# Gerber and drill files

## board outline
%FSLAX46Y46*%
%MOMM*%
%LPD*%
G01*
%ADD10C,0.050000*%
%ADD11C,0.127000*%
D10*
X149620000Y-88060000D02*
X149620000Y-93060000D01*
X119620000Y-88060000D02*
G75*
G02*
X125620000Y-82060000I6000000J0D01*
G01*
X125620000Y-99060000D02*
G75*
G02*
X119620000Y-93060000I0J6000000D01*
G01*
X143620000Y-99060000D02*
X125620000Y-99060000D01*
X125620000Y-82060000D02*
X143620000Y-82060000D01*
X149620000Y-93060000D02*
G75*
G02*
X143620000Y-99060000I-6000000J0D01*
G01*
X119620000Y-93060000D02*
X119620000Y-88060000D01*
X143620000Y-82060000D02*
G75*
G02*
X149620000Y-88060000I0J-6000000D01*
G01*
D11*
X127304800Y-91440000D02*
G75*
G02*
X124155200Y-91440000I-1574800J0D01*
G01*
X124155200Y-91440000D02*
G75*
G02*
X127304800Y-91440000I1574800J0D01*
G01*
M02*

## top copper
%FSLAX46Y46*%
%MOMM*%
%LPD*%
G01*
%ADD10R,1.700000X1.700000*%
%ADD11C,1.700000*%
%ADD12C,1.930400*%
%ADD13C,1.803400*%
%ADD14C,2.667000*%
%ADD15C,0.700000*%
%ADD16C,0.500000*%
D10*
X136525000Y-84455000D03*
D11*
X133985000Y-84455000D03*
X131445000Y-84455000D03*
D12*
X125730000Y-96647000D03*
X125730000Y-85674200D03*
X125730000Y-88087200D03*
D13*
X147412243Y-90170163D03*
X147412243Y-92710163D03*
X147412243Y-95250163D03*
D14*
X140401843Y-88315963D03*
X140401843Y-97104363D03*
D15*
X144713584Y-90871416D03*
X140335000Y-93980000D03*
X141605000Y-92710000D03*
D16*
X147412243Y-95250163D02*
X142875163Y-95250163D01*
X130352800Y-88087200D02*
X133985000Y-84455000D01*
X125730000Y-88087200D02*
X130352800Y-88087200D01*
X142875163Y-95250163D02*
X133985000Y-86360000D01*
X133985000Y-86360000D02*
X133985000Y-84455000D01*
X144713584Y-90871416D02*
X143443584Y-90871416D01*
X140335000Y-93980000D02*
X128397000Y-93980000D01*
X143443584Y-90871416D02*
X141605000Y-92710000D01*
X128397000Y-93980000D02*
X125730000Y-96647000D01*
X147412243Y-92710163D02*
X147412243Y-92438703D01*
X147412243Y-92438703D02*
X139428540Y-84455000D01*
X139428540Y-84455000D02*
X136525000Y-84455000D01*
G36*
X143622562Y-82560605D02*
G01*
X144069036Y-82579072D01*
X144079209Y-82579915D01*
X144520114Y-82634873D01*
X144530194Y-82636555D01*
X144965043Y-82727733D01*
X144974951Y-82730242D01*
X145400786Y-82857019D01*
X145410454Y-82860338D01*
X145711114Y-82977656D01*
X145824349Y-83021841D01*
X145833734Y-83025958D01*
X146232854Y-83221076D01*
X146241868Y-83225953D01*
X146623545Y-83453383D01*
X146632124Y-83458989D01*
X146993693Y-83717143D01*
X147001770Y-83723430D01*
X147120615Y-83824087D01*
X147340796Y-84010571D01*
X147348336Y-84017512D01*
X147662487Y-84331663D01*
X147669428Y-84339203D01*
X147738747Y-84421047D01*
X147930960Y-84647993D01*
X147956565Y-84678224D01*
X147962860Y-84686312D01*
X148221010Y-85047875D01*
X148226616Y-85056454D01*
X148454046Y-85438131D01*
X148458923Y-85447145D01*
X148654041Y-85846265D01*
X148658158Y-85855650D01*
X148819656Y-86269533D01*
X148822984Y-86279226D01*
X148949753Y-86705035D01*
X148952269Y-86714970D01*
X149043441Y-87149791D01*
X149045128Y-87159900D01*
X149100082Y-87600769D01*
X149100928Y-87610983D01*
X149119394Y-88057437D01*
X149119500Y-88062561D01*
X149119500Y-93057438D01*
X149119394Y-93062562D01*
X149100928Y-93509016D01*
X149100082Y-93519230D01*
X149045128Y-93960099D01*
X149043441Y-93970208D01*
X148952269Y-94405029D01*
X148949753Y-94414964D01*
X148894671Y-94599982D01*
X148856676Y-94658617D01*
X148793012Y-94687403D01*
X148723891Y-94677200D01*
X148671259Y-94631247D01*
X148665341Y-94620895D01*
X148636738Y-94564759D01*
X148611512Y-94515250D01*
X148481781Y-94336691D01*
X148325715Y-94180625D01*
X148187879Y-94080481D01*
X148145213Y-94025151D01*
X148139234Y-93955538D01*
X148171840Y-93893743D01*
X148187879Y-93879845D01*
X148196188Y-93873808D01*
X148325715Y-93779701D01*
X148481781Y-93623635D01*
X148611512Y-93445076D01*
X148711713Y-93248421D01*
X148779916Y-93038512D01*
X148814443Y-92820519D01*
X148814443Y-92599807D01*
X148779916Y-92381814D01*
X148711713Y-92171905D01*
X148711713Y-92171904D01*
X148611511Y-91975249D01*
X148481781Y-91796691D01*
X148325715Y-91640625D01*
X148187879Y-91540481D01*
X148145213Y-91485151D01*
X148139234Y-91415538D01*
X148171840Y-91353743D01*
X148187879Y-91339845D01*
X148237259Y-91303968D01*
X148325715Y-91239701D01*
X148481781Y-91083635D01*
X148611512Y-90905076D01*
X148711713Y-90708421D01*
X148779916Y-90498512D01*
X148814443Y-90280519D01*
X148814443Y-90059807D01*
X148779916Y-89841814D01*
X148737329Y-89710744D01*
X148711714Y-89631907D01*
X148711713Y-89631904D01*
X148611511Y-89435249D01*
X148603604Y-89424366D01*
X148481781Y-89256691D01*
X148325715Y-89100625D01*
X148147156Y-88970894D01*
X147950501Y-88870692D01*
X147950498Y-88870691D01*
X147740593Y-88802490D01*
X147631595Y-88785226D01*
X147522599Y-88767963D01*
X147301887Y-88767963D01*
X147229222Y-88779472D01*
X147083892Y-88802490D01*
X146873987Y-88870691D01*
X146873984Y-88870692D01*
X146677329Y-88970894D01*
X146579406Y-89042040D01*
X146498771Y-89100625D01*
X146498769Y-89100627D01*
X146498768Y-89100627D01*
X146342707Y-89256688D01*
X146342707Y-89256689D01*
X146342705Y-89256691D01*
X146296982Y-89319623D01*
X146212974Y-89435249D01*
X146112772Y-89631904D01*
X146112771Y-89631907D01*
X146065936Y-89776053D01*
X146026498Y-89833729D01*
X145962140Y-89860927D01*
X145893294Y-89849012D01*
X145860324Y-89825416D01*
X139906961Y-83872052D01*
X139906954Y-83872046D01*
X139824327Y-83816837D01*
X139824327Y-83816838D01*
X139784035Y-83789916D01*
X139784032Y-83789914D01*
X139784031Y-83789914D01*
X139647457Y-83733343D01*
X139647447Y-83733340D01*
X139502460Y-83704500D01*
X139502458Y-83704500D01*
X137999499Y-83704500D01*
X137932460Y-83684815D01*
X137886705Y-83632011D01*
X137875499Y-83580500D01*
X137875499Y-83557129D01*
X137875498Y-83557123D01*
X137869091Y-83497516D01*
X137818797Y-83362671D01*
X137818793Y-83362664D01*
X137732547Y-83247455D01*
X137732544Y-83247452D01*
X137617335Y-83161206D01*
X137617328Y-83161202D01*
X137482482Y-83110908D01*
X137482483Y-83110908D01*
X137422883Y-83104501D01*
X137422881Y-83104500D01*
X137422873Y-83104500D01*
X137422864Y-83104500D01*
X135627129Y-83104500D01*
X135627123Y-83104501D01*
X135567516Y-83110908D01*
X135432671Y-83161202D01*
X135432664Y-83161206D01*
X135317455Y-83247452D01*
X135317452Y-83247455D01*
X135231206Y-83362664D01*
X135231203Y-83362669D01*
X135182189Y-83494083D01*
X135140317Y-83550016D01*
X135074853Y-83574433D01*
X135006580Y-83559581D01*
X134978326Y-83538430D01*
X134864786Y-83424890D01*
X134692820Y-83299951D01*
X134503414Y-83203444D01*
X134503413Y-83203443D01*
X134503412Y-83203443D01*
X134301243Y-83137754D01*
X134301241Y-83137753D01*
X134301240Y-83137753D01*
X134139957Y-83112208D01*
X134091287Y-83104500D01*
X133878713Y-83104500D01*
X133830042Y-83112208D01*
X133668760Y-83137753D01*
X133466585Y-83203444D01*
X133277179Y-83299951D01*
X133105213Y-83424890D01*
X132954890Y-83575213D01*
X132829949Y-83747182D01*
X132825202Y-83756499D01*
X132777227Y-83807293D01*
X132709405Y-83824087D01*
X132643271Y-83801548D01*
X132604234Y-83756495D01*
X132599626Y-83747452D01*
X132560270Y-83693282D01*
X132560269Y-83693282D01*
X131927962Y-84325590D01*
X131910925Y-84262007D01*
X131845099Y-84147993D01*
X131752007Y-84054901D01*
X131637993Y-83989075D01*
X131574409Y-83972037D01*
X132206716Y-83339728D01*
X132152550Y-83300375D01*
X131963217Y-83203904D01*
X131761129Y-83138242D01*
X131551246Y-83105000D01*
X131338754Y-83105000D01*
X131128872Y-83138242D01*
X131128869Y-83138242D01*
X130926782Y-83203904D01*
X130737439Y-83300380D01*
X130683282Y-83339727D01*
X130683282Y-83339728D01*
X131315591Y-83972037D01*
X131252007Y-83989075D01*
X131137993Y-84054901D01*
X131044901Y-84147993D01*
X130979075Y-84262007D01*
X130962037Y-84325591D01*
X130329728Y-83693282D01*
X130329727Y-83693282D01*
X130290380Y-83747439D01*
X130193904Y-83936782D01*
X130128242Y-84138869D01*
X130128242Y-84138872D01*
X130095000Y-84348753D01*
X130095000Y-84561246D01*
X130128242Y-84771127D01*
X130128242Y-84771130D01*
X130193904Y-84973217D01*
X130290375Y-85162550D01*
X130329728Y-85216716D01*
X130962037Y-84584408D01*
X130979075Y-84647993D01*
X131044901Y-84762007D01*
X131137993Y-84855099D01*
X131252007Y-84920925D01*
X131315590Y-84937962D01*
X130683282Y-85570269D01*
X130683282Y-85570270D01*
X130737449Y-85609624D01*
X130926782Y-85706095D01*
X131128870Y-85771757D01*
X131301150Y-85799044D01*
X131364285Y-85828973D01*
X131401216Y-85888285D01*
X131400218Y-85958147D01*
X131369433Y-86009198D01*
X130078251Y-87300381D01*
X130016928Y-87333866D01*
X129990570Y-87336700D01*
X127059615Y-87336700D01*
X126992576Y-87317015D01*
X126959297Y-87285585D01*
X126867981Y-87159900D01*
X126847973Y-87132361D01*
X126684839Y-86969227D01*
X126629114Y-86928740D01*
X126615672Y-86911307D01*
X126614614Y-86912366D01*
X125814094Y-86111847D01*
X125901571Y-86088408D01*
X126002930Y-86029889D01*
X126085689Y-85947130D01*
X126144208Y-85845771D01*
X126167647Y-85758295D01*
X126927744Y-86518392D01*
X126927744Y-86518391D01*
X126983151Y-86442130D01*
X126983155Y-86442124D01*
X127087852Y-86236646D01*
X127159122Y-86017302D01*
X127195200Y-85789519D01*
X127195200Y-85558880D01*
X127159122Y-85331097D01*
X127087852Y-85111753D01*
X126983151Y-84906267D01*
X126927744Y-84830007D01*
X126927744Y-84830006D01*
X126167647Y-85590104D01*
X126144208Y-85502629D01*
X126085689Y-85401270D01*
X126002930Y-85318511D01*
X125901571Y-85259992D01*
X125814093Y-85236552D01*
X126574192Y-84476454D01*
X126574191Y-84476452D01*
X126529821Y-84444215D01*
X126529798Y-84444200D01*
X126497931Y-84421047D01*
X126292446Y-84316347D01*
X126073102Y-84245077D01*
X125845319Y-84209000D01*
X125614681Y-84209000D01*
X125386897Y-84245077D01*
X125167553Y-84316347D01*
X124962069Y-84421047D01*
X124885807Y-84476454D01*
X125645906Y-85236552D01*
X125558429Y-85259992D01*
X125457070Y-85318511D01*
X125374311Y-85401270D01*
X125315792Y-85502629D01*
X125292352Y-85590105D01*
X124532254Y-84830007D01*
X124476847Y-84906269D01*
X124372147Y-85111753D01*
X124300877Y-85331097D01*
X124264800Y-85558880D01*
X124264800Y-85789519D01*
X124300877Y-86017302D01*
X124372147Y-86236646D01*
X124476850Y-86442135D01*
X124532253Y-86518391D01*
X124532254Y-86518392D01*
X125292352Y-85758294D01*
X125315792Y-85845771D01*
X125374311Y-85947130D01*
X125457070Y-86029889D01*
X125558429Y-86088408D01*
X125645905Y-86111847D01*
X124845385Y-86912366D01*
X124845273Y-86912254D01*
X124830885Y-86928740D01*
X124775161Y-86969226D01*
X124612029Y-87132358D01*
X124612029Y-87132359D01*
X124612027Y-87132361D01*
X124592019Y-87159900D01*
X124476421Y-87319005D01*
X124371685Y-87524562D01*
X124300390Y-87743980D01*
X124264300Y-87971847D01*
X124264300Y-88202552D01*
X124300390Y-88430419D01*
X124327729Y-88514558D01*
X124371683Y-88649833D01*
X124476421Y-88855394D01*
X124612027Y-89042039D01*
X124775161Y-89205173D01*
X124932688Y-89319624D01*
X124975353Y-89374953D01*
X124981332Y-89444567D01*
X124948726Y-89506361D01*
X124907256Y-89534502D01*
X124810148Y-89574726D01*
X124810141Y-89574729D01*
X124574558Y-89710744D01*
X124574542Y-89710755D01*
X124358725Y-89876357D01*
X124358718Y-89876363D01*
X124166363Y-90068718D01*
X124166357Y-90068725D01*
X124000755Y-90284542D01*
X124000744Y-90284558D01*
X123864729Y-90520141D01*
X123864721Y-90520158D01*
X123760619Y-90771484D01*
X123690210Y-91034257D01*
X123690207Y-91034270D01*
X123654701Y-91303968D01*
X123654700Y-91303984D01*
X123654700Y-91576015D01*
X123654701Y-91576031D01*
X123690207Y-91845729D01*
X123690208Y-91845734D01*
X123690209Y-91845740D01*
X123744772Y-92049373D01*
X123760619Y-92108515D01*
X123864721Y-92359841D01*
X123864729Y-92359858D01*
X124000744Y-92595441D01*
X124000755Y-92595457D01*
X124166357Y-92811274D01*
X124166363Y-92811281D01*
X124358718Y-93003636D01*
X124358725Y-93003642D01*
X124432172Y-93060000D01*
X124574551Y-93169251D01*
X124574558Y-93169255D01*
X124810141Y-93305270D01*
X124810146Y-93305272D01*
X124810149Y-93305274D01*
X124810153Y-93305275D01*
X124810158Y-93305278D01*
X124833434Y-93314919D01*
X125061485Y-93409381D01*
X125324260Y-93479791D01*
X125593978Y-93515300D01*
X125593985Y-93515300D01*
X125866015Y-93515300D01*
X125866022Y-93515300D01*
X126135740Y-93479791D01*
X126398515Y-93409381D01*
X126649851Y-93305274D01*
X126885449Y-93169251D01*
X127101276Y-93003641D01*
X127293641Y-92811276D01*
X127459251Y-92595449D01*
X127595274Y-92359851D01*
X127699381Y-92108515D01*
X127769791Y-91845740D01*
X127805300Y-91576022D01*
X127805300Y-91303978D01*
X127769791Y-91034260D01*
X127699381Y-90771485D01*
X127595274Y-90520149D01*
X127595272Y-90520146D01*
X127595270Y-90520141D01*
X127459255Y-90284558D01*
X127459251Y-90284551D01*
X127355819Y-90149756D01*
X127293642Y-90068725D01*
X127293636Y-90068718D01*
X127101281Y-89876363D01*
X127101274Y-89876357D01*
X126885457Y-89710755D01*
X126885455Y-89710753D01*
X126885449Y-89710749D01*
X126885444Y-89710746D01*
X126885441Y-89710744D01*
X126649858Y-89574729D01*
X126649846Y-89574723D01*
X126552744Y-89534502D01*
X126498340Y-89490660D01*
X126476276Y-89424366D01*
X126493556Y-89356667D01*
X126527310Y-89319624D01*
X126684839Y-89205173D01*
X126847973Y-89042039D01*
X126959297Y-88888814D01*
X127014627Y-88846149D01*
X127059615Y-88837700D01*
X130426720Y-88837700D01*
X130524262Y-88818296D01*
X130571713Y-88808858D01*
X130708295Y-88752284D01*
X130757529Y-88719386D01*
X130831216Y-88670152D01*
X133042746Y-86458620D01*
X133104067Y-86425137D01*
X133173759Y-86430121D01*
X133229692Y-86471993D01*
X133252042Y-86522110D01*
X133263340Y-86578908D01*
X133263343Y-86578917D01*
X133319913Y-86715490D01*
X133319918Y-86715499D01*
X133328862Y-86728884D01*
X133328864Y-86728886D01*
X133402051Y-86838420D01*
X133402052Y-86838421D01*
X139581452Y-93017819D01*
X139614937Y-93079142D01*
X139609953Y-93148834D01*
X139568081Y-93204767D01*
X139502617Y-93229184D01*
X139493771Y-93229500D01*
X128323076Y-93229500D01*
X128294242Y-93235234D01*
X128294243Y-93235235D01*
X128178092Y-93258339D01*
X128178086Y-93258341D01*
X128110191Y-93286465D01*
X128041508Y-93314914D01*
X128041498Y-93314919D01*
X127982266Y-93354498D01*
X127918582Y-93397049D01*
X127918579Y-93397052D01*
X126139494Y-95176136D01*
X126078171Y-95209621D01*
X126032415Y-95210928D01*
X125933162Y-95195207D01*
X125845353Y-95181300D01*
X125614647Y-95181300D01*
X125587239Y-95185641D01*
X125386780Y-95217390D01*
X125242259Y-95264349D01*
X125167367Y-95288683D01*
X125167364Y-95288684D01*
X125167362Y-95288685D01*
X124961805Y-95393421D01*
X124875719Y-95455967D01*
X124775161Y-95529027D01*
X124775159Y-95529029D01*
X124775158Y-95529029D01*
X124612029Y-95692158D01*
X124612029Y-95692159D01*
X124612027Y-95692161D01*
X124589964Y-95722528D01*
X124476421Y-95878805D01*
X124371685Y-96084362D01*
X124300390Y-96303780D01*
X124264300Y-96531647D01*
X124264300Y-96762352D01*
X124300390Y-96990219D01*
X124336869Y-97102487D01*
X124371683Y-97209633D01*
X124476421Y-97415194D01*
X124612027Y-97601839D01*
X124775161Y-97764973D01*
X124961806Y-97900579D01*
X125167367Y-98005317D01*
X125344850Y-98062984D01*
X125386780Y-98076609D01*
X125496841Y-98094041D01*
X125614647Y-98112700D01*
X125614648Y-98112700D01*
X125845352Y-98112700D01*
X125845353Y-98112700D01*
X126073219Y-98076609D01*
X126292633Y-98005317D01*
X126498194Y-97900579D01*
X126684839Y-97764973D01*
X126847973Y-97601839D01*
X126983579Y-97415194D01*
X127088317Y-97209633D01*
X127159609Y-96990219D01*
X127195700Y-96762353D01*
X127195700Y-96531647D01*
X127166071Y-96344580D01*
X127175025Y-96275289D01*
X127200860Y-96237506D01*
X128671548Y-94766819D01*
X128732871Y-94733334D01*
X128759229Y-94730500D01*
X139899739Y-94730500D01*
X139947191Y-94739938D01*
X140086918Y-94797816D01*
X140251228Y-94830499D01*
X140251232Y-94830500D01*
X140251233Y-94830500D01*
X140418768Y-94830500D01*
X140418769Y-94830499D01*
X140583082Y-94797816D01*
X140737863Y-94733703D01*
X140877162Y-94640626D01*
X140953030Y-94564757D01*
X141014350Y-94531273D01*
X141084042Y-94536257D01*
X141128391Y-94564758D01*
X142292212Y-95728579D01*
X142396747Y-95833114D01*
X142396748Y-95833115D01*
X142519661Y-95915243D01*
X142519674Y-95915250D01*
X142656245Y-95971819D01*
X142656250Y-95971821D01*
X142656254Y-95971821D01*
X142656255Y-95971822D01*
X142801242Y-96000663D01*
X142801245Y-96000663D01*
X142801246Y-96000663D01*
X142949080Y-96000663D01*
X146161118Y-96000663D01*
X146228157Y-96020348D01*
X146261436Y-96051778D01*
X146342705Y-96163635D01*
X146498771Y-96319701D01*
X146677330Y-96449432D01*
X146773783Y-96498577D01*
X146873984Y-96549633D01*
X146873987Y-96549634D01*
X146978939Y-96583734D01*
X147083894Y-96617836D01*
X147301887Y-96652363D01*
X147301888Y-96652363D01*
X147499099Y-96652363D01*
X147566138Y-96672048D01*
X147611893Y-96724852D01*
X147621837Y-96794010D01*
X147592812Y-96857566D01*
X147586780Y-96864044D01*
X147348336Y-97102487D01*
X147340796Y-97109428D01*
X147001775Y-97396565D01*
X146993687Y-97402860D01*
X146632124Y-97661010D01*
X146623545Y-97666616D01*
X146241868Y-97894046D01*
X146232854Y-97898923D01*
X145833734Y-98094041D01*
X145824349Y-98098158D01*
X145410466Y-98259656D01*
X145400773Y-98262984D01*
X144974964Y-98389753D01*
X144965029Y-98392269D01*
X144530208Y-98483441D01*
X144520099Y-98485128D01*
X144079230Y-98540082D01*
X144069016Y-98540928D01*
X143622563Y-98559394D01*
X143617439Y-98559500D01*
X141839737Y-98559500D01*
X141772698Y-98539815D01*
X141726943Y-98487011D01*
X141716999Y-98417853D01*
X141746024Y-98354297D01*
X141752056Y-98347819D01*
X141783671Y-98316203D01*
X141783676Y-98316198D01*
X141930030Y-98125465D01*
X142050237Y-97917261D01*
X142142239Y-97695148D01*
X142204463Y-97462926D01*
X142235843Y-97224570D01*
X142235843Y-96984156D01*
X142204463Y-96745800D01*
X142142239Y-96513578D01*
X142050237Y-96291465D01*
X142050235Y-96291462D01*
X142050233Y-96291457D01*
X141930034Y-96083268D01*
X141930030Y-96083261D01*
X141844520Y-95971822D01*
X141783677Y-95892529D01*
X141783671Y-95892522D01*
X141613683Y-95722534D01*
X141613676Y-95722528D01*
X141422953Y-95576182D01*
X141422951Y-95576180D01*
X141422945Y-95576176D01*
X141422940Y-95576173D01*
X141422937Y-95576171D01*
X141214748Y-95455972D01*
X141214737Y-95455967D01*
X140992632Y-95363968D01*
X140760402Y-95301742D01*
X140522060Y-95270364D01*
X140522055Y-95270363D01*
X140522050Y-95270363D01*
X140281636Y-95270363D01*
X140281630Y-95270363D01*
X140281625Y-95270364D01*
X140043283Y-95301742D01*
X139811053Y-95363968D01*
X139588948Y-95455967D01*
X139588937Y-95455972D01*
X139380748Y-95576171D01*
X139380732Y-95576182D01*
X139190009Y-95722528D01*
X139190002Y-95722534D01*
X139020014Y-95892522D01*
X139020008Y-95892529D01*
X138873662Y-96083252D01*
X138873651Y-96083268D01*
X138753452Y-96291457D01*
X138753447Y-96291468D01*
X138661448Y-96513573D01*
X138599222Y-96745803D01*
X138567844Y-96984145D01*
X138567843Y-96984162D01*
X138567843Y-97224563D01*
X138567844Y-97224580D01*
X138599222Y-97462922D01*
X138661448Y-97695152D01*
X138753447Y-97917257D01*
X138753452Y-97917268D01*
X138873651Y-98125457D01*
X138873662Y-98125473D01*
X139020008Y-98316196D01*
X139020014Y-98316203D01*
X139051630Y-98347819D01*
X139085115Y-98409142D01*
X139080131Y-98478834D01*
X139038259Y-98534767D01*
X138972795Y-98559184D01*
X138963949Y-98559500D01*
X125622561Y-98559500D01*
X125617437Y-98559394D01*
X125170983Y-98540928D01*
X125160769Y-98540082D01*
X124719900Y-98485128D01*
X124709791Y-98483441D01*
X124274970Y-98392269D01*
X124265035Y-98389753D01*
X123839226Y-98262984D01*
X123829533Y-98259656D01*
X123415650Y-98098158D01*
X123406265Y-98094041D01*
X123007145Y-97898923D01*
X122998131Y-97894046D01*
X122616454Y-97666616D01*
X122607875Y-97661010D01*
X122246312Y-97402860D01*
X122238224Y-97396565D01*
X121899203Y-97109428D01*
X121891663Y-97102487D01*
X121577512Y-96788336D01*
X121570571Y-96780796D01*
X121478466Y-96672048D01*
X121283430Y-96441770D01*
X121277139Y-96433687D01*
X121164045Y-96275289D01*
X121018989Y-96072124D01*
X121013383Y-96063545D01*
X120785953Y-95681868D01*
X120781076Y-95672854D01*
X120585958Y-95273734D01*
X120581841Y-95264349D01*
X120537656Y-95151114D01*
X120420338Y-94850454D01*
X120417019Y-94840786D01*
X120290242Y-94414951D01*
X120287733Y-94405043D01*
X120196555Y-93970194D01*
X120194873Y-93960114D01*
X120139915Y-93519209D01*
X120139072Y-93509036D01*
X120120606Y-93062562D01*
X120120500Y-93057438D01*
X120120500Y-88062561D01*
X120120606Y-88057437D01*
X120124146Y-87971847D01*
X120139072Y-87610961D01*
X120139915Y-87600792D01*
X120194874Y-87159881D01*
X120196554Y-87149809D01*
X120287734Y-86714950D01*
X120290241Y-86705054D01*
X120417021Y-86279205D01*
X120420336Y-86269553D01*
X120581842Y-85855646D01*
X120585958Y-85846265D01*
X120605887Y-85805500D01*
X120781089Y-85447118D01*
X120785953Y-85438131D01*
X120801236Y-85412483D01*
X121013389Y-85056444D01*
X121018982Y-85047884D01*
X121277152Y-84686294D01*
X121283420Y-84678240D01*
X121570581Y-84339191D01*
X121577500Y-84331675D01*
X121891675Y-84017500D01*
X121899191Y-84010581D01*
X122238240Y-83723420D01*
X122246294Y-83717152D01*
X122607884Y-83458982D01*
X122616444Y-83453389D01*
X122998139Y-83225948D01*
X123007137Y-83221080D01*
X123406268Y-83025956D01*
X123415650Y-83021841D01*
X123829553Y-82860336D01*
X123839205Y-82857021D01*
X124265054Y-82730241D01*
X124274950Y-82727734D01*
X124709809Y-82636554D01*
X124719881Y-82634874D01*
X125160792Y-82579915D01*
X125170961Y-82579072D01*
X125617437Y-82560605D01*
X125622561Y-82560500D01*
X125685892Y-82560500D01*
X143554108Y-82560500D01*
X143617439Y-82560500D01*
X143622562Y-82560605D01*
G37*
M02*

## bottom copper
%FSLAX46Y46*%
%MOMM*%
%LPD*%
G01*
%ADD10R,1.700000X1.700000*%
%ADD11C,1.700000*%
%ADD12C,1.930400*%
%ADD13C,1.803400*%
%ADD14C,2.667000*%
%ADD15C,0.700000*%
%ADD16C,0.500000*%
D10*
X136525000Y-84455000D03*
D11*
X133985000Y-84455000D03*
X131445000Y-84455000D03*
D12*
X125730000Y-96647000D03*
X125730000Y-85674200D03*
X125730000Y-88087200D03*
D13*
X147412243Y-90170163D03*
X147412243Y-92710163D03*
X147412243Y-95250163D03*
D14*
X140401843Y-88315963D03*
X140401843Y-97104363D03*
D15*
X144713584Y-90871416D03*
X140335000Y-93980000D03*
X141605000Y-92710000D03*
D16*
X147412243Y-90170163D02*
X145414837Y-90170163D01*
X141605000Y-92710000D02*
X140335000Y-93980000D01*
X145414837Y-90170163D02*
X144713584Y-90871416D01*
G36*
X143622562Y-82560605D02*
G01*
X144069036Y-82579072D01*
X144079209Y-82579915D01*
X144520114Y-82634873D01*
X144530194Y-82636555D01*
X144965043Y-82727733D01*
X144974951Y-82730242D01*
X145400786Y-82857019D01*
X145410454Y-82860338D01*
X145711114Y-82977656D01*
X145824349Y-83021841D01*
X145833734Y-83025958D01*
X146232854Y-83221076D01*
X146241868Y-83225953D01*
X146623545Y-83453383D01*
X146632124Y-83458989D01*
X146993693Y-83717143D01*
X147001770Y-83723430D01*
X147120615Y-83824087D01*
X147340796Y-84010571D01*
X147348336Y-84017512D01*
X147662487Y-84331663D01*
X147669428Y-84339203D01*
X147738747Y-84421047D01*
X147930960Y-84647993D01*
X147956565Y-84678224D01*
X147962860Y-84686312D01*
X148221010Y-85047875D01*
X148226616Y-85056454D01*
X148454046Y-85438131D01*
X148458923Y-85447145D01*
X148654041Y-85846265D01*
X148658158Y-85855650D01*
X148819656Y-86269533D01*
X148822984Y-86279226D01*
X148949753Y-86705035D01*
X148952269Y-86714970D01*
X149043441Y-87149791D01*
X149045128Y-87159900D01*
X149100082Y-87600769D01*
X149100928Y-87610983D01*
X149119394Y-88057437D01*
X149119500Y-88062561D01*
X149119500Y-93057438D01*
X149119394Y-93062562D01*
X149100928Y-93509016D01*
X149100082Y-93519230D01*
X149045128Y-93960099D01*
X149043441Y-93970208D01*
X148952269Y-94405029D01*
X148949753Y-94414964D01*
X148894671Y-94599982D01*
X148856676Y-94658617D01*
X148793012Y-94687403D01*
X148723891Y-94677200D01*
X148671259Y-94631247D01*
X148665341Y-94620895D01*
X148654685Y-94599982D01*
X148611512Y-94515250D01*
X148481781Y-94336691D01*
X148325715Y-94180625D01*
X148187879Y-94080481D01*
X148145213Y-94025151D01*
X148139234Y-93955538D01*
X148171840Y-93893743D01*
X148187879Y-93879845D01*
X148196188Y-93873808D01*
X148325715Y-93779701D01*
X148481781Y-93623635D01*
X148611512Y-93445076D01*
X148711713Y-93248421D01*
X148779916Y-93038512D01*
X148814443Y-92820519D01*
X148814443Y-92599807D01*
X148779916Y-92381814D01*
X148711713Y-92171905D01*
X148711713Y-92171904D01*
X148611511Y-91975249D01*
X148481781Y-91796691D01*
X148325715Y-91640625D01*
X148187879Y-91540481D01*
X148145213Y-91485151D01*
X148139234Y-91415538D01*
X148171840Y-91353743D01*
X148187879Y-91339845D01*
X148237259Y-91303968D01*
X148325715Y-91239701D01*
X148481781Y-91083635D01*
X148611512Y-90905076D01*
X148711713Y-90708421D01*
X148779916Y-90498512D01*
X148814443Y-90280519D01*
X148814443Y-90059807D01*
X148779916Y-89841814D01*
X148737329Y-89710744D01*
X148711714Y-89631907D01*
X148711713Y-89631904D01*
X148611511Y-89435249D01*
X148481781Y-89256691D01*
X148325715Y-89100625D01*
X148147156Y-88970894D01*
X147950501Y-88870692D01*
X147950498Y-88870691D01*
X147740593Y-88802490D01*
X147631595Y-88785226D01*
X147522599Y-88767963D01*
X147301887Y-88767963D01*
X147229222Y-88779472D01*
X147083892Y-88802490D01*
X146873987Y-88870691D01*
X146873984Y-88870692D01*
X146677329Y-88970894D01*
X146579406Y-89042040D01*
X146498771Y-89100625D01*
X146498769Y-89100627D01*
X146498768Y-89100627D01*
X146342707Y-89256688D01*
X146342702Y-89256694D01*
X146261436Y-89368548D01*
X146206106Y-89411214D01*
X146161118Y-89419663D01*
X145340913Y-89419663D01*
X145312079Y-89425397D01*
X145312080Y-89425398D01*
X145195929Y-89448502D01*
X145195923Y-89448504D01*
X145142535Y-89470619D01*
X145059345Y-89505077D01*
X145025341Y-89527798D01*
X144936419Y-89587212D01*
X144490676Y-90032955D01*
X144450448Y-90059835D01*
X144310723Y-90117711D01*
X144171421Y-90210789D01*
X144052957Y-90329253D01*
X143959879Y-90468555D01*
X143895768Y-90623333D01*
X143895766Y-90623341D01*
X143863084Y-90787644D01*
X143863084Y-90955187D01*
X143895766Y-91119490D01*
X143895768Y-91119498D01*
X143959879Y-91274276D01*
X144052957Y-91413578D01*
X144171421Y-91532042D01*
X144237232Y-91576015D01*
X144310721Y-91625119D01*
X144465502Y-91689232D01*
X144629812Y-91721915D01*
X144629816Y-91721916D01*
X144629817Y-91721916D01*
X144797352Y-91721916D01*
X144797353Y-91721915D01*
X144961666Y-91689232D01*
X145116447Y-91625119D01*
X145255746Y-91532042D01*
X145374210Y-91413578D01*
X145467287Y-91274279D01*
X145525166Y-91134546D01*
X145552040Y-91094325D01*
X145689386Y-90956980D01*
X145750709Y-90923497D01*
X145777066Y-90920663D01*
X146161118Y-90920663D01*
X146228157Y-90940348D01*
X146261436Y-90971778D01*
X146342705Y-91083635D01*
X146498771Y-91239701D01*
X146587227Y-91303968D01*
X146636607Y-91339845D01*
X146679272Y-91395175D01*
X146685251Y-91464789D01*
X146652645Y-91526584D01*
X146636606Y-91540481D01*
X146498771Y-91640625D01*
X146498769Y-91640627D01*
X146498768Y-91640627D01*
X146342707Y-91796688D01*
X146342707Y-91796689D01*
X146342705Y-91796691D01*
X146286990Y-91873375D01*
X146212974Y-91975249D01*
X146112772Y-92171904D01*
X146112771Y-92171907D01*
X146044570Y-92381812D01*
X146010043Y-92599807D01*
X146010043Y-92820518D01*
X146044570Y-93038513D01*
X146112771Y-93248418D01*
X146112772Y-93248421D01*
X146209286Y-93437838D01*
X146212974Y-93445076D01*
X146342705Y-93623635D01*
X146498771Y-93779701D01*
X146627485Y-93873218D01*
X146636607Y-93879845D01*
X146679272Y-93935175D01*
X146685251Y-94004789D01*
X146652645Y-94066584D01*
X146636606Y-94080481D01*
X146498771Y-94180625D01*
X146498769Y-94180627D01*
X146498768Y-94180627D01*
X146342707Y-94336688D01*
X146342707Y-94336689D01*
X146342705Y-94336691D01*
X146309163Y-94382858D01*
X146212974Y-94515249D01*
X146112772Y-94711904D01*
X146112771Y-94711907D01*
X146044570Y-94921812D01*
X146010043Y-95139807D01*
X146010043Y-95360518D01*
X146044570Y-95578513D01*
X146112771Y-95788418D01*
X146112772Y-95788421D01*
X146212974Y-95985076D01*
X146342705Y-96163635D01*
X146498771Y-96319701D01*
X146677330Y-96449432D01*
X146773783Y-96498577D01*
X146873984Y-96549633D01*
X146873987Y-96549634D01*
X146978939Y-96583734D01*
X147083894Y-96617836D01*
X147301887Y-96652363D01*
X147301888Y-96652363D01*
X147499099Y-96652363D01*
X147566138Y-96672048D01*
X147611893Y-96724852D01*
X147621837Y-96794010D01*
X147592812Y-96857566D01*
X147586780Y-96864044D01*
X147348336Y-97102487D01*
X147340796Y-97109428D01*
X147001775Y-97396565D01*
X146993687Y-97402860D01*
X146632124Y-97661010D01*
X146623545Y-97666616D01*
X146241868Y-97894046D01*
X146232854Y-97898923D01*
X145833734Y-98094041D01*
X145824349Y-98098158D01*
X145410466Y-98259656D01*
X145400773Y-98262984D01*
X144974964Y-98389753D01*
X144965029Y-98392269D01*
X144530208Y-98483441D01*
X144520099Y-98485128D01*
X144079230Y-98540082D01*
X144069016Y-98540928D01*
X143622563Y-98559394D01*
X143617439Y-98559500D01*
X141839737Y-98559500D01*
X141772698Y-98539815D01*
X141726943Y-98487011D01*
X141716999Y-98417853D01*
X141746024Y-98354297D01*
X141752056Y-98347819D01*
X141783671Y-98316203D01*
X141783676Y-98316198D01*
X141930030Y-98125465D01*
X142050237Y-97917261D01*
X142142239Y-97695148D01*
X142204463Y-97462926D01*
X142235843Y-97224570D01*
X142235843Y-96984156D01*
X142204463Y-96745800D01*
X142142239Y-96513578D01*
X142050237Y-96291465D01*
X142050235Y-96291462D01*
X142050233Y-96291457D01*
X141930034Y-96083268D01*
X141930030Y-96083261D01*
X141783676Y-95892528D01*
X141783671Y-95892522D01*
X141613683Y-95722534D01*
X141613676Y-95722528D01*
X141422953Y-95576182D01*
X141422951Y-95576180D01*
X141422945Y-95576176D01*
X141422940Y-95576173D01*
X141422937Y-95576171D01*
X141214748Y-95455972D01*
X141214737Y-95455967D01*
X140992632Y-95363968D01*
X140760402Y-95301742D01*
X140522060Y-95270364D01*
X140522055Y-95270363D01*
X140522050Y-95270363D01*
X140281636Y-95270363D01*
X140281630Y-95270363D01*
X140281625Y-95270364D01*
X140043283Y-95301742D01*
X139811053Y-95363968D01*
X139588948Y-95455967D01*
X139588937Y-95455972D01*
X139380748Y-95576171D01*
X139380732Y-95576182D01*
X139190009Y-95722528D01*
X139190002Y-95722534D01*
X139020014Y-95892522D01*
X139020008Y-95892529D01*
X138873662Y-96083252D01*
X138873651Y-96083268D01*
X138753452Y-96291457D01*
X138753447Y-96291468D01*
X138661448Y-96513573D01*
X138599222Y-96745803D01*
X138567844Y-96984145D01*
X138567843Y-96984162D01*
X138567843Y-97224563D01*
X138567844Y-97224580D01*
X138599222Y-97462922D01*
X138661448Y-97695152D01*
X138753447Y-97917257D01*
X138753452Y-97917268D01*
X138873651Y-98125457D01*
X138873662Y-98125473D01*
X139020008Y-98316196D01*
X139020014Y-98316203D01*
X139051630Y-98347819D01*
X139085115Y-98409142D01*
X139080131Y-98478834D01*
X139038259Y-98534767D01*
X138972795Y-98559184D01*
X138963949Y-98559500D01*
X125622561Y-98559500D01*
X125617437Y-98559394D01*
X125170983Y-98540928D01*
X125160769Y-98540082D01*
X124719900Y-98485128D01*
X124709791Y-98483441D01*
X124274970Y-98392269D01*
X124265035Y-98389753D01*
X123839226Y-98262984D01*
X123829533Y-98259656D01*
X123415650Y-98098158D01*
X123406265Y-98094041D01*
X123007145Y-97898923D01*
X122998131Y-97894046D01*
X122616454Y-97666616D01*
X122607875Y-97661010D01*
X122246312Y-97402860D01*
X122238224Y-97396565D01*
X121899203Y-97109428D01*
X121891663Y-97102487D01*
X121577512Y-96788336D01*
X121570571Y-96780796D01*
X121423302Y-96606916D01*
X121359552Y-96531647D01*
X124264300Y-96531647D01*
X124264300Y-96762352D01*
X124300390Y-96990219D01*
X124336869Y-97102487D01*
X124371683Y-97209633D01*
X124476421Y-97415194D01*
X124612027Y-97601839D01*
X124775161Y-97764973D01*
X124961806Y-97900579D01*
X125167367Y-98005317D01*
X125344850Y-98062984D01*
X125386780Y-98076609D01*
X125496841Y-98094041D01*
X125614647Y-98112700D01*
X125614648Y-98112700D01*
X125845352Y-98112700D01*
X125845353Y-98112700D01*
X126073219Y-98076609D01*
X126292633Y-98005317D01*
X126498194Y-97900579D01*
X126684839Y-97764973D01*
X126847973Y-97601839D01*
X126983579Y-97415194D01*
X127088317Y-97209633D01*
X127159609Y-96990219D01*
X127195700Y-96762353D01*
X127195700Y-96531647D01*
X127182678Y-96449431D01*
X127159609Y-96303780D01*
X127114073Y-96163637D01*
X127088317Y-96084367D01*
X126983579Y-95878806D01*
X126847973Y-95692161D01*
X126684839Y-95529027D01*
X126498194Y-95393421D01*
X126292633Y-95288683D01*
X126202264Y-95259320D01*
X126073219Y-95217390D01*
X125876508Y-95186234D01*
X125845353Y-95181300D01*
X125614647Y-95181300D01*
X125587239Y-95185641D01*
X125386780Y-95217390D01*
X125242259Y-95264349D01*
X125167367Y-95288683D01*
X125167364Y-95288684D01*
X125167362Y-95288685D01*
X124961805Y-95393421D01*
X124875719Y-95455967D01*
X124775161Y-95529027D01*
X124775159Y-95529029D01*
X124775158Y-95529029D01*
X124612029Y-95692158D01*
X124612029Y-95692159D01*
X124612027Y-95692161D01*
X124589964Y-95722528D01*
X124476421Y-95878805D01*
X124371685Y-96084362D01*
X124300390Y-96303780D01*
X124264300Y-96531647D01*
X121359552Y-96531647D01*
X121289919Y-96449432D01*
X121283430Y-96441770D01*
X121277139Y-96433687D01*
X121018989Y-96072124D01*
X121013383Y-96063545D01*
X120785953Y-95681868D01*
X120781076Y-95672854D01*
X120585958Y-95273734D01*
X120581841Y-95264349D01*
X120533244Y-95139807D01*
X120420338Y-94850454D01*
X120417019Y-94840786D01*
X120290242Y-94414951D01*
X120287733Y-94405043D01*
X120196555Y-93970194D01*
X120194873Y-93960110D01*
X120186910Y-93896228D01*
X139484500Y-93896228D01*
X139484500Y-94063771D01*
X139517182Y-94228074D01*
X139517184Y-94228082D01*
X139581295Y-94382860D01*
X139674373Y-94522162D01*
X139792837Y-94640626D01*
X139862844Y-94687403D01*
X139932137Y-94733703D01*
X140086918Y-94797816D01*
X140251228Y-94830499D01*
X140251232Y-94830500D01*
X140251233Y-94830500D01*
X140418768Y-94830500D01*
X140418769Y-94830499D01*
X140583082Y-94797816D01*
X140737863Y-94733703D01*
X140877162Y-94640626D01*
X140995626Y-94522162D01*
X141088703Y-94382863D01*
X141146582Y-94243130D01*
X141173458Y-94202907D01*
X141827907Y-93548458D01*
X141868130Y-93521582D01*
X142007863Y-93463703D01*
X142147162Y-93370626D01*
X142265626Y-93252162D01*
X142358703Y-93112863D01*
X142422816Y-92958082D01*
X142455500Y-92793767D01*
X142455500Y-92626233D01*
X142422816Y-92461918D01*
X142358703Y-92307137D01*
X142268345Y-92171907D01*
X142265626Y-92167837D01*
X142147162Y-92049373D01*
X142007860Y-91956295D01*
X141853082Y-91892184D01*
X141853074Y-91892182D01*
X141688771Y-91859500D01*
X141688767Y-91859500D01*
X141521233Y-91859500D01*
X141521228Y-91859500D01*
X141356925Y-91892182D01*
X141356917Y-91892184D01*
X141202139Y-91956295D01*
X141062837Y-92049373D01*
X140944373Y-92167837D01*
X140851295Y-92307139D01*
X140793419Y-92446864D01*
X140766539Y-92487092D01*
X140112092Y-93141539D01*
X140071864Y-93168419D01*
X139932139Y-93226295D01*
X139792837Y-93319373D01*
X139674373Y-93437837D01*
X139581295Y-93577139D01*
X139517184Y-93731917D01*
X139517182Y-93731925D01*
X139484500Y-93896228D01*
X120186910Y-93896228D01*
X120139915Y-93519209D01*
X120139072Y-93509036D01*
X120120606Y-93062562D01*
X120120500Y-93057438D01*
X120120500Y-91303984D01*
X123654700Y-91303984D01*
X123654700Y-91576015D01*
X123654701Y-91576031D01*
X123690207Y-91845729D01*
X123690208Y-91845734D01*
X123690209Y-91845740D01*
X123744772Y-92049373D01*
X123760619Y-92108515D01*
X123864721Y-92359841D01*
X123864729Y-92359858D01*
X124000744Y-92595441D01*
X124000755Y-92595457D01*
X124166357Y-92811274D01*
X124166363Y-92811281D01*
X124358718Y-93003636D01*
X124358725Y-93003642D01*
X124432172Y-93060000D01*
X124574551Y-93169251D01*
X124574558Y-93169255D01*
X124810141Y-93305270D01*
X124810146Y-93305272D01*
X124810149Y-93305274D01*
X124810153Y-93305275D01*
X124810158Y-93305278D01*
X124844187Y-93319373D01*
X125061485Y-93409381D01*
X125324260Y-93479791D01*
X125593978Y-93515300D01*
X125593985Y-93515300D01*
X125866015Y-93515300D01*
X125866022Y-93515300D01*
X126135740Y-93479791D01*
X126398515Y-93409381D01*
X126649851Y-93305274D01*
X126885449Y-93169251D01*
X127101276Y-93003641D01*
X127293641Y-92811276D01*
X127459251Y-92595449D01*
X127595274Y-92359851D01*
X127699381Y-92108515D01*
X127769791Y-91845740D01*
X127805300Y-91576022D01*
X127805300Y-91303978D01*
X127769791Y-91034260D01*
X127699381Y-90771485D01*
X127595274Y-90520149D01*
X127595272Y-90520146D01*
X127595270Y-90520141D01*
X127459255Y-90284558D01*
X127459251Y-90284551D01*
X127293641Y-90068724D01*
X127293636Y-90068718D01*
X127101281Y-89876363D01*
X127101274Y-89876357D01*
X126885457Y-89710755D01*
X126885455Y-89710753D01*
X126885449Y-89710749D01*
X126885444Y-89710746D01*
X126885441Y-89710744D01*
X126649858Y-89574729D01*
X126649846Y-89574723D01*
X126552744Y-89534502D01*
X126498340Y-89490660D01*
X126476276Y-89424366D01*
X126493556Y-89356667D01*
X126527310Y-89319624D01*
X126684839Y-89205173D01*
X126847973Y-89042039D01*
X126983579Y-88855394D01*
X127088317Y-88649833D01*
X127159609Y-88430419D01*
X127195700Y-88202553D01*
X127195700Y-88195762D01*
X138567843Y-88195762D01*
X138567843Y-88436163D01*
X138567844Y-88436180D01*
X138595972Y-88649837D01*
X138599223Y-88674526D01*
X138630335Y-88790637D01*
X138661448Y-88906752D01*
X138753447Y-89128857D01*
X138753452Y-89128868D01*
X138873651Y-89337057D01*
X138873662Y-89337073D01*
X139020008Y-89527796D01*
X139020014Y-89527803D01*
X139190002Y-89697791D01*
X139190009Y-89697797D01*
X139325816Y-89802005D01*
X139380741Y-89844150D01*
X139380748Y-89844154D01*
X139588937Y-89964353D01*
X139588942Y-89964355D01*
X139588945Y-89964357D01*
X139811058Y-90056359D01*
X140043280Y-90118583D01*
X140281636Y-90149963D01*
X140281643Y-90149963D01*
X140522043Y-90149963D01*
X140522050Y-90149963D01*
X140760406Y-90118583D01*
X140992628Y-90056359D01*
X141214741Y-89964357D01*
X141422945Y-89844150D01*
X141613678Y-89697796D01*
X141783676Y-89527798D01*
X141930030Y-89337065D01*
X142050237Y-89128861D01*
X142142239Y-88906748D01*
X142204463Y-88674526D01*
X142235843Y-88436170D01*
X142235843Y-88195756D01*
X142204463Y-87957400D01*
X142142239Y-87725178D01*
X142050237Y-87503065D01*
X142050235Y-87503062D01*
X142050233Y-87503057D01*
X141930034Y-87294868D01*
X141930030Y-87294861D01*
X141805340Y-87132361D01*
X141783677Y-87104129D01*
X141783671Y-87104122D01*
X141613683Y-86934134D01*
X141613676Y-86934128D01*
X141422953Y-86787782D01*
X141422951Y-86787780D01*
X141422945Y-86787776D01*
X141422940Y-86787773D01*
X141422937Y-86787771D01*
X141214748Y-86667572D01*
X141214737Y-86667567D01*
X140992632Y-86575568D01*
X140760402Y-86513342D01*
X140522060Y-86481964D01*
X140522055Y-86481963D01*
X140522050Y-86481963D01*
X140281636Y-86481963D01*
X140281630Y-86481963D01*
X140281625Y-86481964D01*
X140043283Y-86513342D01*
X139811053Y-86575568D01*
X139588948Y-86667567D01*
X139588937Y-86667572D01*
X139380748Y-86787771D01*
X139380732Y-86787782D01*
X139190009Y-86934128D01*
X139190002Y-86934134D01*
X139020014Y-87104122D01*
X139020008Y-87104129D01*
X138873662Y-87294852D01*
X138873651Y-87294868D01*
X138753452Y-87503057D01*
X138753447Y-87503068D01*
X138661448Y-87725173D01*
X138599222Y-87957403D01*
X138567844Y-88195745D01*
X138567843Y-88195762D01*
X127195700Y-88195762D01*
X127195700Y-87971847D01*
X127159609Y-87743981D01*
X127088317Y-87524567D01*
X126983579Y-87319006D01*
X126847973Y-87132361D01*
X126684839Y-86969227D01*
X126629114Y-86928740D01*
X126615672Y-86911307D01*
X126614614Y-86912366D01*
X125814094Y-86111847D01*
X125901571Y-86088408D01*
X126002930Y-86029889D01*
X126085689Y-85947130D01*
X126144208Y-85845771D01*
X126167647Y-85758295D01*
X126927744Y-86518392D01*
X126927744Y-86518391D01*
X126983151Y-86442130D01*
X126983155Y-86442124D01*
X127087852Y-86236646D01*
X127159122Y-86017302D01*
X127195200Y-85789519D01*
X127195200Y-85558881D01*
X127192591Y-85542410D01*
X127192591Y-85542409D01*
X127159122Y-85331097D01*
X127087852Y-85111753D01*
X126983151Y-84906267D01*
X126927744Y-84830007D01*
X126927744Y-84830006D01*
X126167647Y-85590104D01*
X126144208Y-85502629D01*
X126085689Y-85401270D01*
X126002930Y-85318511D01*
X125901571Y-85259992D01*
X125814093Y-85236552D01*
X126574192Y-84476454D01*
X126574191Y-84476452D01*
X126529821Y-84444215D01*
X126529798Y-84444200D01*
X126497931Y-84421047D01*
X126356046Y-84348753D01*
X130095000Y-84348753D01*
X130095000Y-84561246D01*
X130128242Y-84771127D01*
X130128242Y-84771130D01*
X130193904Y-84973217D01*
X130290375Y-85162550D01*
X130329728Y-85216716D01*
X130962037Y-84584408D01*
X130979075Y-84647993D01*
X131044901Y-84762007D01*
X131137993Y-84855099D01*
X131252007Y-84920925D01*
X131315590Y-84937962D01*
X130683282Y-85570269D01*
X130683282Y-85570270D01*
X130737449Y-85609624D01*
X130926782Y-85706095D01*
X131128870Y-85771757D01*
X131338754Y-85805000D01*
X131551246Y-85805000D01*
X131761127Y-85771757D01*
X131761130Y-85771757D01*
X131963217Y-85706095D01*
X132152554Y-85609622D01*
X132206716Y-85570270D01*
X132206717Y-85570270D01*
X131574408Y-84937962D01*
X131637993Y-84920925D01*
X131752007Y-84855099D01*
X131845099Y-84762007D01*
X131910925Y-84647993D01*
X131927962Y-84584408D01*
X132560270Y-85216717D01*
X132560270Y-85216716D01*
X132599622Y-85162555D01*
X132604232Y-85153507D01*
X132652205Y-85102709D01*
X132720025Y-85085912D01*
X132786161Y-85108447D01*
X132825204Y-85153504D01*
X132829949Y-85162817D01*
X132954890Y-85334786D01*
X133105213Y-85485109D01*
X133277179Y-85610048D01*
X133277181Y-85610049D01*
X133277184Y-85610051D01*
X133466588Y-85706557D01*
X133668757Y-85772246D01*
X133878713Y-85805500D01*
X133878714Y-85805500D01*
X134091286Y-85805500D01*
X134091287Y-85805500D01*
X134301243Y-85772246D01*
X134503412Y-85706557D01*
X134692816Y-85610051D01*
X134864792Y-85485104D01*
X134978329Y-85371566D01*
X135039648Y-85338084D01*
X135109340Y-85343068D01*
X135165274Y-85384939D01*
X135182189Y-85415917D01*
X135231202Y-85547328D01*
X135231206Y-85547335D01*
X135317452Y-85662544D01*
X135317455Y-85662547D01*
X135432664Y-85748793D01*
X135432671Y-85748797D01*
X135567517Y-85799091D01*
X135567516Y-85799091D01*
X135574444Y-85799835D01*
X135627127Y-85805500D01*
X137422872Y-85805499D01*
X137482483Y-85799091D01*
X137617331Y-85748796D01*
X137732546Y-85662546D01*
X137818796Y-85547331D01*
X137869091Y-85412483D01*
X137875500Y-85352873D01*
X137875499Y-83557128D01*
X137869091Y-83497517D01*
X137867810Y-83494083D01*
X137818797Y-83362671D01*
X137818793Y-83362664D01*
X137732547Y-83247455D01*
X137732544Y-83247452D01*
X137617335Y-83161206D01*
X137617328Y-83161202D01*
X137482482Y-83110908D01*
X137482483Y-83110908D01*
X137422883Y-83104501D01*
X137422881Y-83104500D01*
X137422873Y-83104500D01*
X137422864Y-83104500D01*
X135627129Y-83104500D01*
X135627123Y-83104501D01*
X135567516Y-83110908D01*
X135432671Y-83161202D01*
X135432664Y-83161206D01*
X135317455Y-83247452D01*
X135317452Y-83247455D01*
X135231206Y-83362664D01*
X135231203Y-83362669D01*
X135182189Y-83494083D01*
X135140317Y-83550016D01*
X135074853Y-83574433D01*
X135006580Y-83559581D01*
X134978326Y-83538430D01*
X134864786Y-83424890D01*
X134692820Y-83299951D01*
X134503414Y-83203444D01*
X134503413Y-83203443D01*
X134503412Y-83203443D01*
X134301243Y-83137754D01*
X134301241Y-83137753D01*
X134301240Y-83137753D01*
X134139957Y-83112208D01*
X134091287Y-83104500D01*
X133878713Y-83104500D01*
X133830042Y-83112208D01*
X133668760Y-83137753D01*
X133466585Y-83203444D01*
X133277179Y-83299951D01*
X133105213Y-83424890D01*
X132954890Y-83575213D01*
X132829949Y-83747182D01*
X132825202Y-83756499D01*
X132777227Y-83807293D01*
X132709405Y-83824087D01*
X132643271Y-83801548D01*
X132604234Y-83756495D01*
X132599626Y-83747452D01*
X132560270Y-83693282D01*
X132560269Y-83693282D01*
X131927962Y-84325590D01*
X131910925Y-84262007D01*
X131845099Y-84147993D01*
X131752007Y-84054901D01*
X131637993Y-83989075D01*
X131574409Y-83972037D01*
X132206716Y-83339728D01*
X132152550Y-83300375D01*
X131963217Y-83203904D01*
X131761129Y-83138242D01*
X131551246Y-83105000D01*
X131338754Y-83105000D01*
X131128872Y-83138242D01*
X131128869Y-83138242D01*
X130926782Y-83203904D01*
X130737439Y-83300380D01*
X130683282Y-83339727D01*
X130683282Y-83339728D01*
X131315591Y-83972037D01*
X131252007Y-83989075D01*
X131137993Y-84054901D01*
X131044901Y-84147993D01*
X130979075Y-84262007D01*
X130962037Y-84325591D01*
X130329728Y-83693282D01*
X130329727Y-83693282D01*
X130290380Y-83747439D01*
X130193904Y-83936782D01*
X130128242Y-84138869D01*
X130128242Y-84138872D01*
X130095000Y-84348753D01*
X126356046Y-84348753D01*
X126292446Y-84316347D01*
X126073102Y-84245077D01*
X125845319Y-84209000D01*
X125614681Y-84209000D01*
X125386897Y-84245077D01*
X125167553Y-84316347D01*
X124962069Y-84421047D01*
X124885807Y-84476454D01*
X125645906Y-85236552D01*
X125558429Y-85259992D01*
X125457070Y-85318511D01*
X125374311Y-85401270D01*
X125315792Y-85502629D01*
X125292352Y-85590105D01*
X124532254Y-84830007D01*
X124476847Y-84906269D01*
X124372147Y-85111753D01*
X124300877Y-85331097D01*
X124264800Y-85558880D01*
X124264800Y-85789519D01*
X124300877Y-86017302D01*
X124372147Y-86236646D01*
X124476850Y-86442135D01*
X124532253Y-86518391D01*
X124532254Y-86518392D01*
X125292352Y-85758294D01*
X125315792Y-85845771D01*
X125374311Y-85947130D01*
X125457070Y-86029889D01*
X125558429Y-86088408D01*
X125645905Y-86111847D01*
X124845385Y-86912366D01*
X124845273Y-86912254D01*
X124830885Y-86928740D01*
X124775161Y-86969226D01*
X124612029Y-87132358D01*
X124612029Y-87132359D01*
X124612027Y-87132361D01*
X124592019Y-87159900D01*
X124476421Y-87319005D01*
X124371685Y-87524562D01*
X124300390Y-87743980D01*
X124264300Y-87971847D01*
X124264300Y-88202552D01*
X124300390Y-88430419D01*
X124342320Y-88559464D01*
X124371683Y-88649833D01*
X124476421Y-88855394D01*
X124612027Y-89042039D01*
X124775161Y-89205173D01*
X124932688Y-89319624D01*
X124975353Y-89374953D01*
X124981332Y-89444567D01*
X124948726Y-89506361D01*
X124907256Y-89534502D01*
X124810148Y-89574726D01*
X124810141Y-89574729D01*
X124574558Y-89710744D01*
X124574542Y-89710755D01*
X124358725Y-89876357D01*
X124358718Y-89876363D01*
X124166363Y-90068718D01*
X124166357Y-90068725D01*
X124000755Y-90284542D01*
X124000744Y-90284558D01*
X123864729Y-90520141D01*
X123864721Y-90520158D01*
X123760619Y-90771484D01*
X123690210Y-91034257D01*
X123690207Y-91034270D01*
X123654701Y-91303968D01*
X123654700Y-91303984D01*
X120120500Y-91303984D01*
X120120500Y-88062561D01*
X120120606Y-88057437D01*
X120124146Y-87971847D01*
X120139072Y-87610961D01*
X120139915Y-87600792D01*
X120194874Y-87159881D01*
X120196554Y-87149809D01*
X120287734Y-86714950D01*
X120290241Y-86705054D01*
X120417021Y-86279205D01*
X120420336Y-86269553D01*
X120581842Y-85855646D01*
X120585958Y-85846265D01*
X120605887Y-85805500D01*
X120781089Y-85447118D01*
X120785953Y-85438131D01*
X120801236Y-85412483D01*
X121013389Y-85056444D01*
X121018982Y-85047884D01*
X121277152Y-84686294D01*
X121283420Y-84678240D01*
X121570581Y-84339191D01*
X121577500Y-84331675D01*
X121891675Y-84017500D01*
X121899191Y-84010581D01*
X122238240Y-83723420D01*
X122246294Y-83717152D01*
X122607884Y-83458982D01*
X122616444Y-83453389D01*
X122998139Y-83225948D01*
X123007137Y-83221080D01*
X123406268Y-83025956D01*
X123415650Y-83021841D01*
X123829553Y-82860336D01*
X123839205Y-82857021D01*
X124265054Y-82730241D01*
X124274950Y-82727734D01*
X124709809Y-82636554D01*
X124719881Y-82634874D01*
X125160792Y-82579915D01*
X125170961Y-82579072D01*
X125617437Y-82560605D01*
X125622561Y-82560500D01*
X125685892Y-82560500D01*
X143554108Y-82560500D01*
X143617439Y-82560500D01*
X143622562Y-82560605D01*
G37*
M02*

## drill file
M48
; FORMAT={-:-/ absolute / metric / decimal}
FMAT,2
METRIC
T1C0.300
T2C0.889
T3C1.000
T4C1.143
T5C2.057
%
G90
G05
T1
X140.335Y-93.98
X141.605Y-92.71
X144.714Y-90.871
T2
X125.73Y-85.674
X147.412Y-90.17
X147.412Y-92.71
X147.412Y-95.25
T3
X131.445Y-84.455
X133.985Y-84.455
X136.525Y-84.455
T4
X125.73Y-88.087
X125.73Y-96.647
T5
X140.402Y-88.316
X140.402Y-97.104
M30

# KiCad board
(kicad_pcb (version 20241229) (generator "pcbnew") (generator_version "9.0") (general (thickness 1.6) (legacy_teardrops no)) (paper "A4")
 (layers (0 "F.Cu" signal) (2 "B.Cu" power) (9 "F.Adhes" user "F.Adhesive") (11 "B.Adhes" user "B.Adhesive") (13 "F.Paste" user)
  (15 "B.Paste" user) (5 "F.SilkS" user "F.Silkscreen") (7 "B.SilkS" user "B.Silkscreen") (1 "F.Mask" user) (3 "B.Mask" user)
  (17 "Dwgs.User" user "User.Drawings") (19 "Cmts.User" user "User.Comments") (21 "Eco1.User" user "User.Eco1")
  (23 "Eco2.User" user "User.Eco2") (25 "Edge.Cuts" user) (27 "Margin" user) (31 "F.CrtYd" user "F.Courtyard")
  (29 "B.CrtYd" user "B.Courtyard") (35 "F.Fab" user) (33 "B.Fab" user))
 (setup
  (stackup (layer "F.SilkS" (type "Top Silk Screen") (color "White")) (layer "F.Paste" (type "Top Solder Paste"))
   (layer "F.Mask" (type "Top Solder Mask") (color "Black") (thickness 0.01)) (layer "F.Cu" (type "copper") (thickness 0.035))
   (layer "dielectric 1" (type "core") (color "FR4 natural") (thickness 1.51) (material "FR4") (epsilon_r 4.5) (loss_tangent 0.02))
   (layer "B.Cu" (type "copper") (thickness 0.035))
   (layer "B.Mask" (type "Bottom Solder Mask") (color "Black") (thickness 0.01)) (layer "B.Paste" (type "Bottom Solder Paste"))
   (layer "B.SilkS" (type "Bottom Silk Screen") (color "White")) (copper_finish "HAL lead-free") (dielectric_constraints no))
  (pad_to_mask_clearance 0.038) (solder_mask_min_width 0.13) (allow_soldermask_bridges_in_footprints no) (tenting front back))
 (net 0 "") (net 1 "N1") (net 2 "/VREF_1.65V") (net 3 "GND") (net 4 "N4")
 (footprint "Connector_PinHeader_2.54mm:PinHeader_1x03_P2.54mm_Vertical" (layer "F.Cu") (at 136.525 84.455 -90)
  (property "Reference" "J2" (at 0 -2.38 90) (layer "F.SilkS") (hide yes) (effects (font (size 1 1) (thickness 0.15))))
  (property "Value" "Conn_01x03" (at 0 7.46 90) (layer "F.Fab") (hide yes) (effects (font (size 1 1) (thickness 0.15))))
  (pad "1" thru_hole rect (at 0 0 270) (size 1.7 1.7) (drill 1) (layers "*.Cu" "*.Mask") (remove_unused_layers no) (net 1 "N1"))
  (pad "2" thru_hole circle (at 0 2.54 270) (size 1.7 1.7) (drill 1) (layers "*.Cu" "*.Mask") (remove_unused_layers no)
   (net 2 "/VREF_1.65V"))
  (pad "3" thru_hole circle (at 0 5.08 270) (size 1.7 1.7) (drill 1) (layers "*.Cu" "*.Mask") (remove_unused_layers no) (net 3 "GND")))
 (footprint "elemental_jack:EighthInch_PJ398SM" (layer "B.Cu") (at 125.73 91.44 90)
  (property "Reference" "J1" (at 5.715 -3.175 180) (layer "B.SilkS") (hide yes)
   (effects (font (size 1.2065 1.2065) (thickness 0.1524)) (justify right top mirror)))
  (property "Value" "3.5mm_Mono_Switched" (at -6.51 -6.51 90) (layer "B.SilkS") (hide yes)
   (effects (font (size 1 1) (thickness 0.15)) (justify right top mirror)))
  (fp_circle (center 0 0) (end 1.5748 0) (stroke (width 0.127) (type solid)) (fill no) (layer "Edge.Cuts"))
  (pad "1" thru_hole circle (at -5.207 0 90) (size 1.9304 1.9304) (drill 1.143) (layers "*.Cu" "*.Mask") (remove_unused_layers no)
   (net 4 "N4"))
  (pad "2" thru_hole circle (at 5.7658 0 90) (size 1.9304 1.9304) (drill 0.889) (layers "*.Cu" "*.Mask") (remove_unused_layers no)
   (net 3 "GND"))
  (pad "3" thru_hole circle (at 3.3528 0 90) (size 1.9304 1.9304) (drill 1.143) (layers "*.Cu" "*.Mask") (remove_unused_layers no)
   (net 2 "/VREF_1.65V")))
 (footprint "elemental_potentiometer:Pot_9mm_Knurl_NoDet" (layer "B.Cu") (at 140.4 92.71 90)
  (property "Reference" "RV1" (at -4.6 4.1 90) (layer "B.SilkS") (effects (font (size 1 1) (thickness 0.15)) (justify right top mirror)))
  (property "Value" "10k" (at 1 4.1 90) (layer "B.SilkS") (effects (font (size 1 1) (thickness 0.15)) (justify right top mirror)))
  (pad "1" thru_hole circle (at 2.539837 7.012243 180) (size 1.8034 1.8034) (drill 0.889) (layers "*.Cu" "*.Mask") (remove_unused_layers no)
   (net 4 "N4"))
  (pad "2" thru_hole circle (at -0.000163 7.012243 180) (size 1.8034 1.8034) (drill 0.889) (layers "*.Cu" "*.Mask")
   (remove_unused_layers no) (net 1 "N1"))
  (pad "3" thru_hole circle (at -2.540163 7.012243 180) (size 1.8034 1.8034) (drill 0.889) (layers "*.Cu" "*.Mask")
   (remove_unused_layers no) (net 2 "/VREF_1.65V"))
  (pad "4" thru_hole circle (at 4.394037 0.001843 90) (size 2.667 2.667) (drill 2.0574) (layers "*.Cu" "*.Mask") (remove_unused_layers no))
  (pad "5" thru_hole circle (at -4.394363 0.001843 90) (size 2.667 2.667) (drill 2.0574) (layers "*.Cu" "*.Mask") (remove_unused_layers no)))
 (gr_line (start 149.62 88.06) (end 149.62 93.06) (stroke (width 0.05) (type default)) (layer "Edge.Cuts"))
 (gr_arc (start 119.62 88.06) (mid 121.377359 83.817359) (end 125.62 82.06) (stroke (width 0.05) (type default)) (layer "Edge.Cuts"))
 (gr_arc (start 125.62 99.06) (mid 121.377359 97.302641) (end 119.62 93.06) (stroke (width 0.05) (type default)) (layer "Edge.Cuts"))
 (gr_line (start 143.62 99.06) (end 125.62 99.06) (stroke (width 0.05) (type default)) (layer "Edge.Cuts"))
 (gr_line (start 125.62 82.06) (end 143.62 82.06) (stroke (width 0.05) (type default)) (layer "Edge.Cuts"))
 (gr_arc (start 149.62 93.06) (mid 147.862641 97.302641) (end 143.62 99.06) (stroke (width 0.05) (type default)) (layer "Edge.Cuts"))
 (gr_line (start 119.62 93.06) (end 119.62 88.06) (stroke (width 0.05) (type default)) (layer "Edge.Cuts"))
 (gr_arc (start 143.62 82.06) (mid 147.862641 83.817359) (end 149.62 88.06) (stroke (width 0.05) (type default)) (layer "Edge.Cuts"))
 (segment (start 147.412243 95.250163) (end 142.875163 95.250163) (width 0.5) (layer "F.Cu") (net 2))
 (segment (start 130.3528 88.0872) (end 133.985 84.455) (width 0.5) (layer "F.Cu") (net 2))
 (segment (start 125.73 88.0872) (end 130.3528 88.0872) (width 0.5) (layer "F.Cu") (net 2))
 (segment (start 142.875163 95.250163) (end 133.985 86.36) (width 0.5) (layer "F.Cu") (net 2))
 (segment (start 133.985 86.36) (end 133.985 84.455) (width 0.5) (layer "F.Cu") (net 2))
 (segment (start 144.713584 90.871416) (end 143.443584 90.871416) (width 0.5) (layer "F.Cu") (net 4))
 (segment (start 140.335 93.98) (end 128.397 93.98) (width 0.5) (layer "F.Cu") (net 4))
 (segment (start 143.443584 90.871416) (end 141.605 92.71) (width 0.5) (layer "F.Cu") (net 4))
 (segment (start 128.397 93.98) (end 125.73 96.647) (width 0.5) (layer "F.Cu") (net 4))
 (via (at 144.713584 90.871416) (size 0.7) (drill 0.3) (layers "F.Cu" "B.Cu") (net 4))
 (via (at 140.335 93.98) (size 0.7) (drill 0.3) (layers "F.Cu" "B.Cu") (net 4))
 (via (at 141.605 92.71) (size 0.7) (drill 0.3) (layers "F.Cu" "B.Cu") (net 4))
 (segment (start 147.412243 90.170163) (end 145.414837 90.170163) (width 0.5) (layer "B.Cu") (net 4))
 (segment (start 141.605 92.71) (end 140.335 93.98) (width 0.5) (layer "B.Cu") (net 4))
 (segment (start 145.414837 90.170163) (end 144.713584 90.871416) (width 0.5) (layer "B.Cu") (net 4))
 (segment (start 147.412243 92.710163) (end 147.412243 92.438703) (width 0.5) (layer "F.Cu") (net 1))
 (segment (start 147.412243 92.438703) (end 139.42854 84.455) (width 0.5) (layer "F.Cu") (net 1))
 (segment (start 139.42854 84.455) (end 136.525 84.455) (width 0.5) (layer "F.Cu") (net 1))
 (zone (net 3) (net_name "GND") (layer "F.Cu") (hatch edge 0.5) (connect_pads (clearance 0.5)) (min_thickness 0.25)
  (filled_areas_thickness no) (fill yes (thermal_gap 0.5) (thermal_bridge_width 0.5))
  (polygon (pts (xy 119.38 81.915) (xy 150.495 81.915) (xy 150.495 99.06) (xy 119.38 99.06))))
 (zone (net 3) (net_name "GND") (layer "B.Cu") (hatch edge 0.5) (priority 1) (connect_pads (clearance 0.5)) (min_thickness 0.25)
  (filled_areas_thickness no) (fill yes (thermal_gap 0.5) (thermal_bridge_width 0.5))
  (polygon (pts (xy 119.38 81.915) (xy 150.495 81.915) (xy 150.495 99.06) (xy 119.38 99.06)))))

